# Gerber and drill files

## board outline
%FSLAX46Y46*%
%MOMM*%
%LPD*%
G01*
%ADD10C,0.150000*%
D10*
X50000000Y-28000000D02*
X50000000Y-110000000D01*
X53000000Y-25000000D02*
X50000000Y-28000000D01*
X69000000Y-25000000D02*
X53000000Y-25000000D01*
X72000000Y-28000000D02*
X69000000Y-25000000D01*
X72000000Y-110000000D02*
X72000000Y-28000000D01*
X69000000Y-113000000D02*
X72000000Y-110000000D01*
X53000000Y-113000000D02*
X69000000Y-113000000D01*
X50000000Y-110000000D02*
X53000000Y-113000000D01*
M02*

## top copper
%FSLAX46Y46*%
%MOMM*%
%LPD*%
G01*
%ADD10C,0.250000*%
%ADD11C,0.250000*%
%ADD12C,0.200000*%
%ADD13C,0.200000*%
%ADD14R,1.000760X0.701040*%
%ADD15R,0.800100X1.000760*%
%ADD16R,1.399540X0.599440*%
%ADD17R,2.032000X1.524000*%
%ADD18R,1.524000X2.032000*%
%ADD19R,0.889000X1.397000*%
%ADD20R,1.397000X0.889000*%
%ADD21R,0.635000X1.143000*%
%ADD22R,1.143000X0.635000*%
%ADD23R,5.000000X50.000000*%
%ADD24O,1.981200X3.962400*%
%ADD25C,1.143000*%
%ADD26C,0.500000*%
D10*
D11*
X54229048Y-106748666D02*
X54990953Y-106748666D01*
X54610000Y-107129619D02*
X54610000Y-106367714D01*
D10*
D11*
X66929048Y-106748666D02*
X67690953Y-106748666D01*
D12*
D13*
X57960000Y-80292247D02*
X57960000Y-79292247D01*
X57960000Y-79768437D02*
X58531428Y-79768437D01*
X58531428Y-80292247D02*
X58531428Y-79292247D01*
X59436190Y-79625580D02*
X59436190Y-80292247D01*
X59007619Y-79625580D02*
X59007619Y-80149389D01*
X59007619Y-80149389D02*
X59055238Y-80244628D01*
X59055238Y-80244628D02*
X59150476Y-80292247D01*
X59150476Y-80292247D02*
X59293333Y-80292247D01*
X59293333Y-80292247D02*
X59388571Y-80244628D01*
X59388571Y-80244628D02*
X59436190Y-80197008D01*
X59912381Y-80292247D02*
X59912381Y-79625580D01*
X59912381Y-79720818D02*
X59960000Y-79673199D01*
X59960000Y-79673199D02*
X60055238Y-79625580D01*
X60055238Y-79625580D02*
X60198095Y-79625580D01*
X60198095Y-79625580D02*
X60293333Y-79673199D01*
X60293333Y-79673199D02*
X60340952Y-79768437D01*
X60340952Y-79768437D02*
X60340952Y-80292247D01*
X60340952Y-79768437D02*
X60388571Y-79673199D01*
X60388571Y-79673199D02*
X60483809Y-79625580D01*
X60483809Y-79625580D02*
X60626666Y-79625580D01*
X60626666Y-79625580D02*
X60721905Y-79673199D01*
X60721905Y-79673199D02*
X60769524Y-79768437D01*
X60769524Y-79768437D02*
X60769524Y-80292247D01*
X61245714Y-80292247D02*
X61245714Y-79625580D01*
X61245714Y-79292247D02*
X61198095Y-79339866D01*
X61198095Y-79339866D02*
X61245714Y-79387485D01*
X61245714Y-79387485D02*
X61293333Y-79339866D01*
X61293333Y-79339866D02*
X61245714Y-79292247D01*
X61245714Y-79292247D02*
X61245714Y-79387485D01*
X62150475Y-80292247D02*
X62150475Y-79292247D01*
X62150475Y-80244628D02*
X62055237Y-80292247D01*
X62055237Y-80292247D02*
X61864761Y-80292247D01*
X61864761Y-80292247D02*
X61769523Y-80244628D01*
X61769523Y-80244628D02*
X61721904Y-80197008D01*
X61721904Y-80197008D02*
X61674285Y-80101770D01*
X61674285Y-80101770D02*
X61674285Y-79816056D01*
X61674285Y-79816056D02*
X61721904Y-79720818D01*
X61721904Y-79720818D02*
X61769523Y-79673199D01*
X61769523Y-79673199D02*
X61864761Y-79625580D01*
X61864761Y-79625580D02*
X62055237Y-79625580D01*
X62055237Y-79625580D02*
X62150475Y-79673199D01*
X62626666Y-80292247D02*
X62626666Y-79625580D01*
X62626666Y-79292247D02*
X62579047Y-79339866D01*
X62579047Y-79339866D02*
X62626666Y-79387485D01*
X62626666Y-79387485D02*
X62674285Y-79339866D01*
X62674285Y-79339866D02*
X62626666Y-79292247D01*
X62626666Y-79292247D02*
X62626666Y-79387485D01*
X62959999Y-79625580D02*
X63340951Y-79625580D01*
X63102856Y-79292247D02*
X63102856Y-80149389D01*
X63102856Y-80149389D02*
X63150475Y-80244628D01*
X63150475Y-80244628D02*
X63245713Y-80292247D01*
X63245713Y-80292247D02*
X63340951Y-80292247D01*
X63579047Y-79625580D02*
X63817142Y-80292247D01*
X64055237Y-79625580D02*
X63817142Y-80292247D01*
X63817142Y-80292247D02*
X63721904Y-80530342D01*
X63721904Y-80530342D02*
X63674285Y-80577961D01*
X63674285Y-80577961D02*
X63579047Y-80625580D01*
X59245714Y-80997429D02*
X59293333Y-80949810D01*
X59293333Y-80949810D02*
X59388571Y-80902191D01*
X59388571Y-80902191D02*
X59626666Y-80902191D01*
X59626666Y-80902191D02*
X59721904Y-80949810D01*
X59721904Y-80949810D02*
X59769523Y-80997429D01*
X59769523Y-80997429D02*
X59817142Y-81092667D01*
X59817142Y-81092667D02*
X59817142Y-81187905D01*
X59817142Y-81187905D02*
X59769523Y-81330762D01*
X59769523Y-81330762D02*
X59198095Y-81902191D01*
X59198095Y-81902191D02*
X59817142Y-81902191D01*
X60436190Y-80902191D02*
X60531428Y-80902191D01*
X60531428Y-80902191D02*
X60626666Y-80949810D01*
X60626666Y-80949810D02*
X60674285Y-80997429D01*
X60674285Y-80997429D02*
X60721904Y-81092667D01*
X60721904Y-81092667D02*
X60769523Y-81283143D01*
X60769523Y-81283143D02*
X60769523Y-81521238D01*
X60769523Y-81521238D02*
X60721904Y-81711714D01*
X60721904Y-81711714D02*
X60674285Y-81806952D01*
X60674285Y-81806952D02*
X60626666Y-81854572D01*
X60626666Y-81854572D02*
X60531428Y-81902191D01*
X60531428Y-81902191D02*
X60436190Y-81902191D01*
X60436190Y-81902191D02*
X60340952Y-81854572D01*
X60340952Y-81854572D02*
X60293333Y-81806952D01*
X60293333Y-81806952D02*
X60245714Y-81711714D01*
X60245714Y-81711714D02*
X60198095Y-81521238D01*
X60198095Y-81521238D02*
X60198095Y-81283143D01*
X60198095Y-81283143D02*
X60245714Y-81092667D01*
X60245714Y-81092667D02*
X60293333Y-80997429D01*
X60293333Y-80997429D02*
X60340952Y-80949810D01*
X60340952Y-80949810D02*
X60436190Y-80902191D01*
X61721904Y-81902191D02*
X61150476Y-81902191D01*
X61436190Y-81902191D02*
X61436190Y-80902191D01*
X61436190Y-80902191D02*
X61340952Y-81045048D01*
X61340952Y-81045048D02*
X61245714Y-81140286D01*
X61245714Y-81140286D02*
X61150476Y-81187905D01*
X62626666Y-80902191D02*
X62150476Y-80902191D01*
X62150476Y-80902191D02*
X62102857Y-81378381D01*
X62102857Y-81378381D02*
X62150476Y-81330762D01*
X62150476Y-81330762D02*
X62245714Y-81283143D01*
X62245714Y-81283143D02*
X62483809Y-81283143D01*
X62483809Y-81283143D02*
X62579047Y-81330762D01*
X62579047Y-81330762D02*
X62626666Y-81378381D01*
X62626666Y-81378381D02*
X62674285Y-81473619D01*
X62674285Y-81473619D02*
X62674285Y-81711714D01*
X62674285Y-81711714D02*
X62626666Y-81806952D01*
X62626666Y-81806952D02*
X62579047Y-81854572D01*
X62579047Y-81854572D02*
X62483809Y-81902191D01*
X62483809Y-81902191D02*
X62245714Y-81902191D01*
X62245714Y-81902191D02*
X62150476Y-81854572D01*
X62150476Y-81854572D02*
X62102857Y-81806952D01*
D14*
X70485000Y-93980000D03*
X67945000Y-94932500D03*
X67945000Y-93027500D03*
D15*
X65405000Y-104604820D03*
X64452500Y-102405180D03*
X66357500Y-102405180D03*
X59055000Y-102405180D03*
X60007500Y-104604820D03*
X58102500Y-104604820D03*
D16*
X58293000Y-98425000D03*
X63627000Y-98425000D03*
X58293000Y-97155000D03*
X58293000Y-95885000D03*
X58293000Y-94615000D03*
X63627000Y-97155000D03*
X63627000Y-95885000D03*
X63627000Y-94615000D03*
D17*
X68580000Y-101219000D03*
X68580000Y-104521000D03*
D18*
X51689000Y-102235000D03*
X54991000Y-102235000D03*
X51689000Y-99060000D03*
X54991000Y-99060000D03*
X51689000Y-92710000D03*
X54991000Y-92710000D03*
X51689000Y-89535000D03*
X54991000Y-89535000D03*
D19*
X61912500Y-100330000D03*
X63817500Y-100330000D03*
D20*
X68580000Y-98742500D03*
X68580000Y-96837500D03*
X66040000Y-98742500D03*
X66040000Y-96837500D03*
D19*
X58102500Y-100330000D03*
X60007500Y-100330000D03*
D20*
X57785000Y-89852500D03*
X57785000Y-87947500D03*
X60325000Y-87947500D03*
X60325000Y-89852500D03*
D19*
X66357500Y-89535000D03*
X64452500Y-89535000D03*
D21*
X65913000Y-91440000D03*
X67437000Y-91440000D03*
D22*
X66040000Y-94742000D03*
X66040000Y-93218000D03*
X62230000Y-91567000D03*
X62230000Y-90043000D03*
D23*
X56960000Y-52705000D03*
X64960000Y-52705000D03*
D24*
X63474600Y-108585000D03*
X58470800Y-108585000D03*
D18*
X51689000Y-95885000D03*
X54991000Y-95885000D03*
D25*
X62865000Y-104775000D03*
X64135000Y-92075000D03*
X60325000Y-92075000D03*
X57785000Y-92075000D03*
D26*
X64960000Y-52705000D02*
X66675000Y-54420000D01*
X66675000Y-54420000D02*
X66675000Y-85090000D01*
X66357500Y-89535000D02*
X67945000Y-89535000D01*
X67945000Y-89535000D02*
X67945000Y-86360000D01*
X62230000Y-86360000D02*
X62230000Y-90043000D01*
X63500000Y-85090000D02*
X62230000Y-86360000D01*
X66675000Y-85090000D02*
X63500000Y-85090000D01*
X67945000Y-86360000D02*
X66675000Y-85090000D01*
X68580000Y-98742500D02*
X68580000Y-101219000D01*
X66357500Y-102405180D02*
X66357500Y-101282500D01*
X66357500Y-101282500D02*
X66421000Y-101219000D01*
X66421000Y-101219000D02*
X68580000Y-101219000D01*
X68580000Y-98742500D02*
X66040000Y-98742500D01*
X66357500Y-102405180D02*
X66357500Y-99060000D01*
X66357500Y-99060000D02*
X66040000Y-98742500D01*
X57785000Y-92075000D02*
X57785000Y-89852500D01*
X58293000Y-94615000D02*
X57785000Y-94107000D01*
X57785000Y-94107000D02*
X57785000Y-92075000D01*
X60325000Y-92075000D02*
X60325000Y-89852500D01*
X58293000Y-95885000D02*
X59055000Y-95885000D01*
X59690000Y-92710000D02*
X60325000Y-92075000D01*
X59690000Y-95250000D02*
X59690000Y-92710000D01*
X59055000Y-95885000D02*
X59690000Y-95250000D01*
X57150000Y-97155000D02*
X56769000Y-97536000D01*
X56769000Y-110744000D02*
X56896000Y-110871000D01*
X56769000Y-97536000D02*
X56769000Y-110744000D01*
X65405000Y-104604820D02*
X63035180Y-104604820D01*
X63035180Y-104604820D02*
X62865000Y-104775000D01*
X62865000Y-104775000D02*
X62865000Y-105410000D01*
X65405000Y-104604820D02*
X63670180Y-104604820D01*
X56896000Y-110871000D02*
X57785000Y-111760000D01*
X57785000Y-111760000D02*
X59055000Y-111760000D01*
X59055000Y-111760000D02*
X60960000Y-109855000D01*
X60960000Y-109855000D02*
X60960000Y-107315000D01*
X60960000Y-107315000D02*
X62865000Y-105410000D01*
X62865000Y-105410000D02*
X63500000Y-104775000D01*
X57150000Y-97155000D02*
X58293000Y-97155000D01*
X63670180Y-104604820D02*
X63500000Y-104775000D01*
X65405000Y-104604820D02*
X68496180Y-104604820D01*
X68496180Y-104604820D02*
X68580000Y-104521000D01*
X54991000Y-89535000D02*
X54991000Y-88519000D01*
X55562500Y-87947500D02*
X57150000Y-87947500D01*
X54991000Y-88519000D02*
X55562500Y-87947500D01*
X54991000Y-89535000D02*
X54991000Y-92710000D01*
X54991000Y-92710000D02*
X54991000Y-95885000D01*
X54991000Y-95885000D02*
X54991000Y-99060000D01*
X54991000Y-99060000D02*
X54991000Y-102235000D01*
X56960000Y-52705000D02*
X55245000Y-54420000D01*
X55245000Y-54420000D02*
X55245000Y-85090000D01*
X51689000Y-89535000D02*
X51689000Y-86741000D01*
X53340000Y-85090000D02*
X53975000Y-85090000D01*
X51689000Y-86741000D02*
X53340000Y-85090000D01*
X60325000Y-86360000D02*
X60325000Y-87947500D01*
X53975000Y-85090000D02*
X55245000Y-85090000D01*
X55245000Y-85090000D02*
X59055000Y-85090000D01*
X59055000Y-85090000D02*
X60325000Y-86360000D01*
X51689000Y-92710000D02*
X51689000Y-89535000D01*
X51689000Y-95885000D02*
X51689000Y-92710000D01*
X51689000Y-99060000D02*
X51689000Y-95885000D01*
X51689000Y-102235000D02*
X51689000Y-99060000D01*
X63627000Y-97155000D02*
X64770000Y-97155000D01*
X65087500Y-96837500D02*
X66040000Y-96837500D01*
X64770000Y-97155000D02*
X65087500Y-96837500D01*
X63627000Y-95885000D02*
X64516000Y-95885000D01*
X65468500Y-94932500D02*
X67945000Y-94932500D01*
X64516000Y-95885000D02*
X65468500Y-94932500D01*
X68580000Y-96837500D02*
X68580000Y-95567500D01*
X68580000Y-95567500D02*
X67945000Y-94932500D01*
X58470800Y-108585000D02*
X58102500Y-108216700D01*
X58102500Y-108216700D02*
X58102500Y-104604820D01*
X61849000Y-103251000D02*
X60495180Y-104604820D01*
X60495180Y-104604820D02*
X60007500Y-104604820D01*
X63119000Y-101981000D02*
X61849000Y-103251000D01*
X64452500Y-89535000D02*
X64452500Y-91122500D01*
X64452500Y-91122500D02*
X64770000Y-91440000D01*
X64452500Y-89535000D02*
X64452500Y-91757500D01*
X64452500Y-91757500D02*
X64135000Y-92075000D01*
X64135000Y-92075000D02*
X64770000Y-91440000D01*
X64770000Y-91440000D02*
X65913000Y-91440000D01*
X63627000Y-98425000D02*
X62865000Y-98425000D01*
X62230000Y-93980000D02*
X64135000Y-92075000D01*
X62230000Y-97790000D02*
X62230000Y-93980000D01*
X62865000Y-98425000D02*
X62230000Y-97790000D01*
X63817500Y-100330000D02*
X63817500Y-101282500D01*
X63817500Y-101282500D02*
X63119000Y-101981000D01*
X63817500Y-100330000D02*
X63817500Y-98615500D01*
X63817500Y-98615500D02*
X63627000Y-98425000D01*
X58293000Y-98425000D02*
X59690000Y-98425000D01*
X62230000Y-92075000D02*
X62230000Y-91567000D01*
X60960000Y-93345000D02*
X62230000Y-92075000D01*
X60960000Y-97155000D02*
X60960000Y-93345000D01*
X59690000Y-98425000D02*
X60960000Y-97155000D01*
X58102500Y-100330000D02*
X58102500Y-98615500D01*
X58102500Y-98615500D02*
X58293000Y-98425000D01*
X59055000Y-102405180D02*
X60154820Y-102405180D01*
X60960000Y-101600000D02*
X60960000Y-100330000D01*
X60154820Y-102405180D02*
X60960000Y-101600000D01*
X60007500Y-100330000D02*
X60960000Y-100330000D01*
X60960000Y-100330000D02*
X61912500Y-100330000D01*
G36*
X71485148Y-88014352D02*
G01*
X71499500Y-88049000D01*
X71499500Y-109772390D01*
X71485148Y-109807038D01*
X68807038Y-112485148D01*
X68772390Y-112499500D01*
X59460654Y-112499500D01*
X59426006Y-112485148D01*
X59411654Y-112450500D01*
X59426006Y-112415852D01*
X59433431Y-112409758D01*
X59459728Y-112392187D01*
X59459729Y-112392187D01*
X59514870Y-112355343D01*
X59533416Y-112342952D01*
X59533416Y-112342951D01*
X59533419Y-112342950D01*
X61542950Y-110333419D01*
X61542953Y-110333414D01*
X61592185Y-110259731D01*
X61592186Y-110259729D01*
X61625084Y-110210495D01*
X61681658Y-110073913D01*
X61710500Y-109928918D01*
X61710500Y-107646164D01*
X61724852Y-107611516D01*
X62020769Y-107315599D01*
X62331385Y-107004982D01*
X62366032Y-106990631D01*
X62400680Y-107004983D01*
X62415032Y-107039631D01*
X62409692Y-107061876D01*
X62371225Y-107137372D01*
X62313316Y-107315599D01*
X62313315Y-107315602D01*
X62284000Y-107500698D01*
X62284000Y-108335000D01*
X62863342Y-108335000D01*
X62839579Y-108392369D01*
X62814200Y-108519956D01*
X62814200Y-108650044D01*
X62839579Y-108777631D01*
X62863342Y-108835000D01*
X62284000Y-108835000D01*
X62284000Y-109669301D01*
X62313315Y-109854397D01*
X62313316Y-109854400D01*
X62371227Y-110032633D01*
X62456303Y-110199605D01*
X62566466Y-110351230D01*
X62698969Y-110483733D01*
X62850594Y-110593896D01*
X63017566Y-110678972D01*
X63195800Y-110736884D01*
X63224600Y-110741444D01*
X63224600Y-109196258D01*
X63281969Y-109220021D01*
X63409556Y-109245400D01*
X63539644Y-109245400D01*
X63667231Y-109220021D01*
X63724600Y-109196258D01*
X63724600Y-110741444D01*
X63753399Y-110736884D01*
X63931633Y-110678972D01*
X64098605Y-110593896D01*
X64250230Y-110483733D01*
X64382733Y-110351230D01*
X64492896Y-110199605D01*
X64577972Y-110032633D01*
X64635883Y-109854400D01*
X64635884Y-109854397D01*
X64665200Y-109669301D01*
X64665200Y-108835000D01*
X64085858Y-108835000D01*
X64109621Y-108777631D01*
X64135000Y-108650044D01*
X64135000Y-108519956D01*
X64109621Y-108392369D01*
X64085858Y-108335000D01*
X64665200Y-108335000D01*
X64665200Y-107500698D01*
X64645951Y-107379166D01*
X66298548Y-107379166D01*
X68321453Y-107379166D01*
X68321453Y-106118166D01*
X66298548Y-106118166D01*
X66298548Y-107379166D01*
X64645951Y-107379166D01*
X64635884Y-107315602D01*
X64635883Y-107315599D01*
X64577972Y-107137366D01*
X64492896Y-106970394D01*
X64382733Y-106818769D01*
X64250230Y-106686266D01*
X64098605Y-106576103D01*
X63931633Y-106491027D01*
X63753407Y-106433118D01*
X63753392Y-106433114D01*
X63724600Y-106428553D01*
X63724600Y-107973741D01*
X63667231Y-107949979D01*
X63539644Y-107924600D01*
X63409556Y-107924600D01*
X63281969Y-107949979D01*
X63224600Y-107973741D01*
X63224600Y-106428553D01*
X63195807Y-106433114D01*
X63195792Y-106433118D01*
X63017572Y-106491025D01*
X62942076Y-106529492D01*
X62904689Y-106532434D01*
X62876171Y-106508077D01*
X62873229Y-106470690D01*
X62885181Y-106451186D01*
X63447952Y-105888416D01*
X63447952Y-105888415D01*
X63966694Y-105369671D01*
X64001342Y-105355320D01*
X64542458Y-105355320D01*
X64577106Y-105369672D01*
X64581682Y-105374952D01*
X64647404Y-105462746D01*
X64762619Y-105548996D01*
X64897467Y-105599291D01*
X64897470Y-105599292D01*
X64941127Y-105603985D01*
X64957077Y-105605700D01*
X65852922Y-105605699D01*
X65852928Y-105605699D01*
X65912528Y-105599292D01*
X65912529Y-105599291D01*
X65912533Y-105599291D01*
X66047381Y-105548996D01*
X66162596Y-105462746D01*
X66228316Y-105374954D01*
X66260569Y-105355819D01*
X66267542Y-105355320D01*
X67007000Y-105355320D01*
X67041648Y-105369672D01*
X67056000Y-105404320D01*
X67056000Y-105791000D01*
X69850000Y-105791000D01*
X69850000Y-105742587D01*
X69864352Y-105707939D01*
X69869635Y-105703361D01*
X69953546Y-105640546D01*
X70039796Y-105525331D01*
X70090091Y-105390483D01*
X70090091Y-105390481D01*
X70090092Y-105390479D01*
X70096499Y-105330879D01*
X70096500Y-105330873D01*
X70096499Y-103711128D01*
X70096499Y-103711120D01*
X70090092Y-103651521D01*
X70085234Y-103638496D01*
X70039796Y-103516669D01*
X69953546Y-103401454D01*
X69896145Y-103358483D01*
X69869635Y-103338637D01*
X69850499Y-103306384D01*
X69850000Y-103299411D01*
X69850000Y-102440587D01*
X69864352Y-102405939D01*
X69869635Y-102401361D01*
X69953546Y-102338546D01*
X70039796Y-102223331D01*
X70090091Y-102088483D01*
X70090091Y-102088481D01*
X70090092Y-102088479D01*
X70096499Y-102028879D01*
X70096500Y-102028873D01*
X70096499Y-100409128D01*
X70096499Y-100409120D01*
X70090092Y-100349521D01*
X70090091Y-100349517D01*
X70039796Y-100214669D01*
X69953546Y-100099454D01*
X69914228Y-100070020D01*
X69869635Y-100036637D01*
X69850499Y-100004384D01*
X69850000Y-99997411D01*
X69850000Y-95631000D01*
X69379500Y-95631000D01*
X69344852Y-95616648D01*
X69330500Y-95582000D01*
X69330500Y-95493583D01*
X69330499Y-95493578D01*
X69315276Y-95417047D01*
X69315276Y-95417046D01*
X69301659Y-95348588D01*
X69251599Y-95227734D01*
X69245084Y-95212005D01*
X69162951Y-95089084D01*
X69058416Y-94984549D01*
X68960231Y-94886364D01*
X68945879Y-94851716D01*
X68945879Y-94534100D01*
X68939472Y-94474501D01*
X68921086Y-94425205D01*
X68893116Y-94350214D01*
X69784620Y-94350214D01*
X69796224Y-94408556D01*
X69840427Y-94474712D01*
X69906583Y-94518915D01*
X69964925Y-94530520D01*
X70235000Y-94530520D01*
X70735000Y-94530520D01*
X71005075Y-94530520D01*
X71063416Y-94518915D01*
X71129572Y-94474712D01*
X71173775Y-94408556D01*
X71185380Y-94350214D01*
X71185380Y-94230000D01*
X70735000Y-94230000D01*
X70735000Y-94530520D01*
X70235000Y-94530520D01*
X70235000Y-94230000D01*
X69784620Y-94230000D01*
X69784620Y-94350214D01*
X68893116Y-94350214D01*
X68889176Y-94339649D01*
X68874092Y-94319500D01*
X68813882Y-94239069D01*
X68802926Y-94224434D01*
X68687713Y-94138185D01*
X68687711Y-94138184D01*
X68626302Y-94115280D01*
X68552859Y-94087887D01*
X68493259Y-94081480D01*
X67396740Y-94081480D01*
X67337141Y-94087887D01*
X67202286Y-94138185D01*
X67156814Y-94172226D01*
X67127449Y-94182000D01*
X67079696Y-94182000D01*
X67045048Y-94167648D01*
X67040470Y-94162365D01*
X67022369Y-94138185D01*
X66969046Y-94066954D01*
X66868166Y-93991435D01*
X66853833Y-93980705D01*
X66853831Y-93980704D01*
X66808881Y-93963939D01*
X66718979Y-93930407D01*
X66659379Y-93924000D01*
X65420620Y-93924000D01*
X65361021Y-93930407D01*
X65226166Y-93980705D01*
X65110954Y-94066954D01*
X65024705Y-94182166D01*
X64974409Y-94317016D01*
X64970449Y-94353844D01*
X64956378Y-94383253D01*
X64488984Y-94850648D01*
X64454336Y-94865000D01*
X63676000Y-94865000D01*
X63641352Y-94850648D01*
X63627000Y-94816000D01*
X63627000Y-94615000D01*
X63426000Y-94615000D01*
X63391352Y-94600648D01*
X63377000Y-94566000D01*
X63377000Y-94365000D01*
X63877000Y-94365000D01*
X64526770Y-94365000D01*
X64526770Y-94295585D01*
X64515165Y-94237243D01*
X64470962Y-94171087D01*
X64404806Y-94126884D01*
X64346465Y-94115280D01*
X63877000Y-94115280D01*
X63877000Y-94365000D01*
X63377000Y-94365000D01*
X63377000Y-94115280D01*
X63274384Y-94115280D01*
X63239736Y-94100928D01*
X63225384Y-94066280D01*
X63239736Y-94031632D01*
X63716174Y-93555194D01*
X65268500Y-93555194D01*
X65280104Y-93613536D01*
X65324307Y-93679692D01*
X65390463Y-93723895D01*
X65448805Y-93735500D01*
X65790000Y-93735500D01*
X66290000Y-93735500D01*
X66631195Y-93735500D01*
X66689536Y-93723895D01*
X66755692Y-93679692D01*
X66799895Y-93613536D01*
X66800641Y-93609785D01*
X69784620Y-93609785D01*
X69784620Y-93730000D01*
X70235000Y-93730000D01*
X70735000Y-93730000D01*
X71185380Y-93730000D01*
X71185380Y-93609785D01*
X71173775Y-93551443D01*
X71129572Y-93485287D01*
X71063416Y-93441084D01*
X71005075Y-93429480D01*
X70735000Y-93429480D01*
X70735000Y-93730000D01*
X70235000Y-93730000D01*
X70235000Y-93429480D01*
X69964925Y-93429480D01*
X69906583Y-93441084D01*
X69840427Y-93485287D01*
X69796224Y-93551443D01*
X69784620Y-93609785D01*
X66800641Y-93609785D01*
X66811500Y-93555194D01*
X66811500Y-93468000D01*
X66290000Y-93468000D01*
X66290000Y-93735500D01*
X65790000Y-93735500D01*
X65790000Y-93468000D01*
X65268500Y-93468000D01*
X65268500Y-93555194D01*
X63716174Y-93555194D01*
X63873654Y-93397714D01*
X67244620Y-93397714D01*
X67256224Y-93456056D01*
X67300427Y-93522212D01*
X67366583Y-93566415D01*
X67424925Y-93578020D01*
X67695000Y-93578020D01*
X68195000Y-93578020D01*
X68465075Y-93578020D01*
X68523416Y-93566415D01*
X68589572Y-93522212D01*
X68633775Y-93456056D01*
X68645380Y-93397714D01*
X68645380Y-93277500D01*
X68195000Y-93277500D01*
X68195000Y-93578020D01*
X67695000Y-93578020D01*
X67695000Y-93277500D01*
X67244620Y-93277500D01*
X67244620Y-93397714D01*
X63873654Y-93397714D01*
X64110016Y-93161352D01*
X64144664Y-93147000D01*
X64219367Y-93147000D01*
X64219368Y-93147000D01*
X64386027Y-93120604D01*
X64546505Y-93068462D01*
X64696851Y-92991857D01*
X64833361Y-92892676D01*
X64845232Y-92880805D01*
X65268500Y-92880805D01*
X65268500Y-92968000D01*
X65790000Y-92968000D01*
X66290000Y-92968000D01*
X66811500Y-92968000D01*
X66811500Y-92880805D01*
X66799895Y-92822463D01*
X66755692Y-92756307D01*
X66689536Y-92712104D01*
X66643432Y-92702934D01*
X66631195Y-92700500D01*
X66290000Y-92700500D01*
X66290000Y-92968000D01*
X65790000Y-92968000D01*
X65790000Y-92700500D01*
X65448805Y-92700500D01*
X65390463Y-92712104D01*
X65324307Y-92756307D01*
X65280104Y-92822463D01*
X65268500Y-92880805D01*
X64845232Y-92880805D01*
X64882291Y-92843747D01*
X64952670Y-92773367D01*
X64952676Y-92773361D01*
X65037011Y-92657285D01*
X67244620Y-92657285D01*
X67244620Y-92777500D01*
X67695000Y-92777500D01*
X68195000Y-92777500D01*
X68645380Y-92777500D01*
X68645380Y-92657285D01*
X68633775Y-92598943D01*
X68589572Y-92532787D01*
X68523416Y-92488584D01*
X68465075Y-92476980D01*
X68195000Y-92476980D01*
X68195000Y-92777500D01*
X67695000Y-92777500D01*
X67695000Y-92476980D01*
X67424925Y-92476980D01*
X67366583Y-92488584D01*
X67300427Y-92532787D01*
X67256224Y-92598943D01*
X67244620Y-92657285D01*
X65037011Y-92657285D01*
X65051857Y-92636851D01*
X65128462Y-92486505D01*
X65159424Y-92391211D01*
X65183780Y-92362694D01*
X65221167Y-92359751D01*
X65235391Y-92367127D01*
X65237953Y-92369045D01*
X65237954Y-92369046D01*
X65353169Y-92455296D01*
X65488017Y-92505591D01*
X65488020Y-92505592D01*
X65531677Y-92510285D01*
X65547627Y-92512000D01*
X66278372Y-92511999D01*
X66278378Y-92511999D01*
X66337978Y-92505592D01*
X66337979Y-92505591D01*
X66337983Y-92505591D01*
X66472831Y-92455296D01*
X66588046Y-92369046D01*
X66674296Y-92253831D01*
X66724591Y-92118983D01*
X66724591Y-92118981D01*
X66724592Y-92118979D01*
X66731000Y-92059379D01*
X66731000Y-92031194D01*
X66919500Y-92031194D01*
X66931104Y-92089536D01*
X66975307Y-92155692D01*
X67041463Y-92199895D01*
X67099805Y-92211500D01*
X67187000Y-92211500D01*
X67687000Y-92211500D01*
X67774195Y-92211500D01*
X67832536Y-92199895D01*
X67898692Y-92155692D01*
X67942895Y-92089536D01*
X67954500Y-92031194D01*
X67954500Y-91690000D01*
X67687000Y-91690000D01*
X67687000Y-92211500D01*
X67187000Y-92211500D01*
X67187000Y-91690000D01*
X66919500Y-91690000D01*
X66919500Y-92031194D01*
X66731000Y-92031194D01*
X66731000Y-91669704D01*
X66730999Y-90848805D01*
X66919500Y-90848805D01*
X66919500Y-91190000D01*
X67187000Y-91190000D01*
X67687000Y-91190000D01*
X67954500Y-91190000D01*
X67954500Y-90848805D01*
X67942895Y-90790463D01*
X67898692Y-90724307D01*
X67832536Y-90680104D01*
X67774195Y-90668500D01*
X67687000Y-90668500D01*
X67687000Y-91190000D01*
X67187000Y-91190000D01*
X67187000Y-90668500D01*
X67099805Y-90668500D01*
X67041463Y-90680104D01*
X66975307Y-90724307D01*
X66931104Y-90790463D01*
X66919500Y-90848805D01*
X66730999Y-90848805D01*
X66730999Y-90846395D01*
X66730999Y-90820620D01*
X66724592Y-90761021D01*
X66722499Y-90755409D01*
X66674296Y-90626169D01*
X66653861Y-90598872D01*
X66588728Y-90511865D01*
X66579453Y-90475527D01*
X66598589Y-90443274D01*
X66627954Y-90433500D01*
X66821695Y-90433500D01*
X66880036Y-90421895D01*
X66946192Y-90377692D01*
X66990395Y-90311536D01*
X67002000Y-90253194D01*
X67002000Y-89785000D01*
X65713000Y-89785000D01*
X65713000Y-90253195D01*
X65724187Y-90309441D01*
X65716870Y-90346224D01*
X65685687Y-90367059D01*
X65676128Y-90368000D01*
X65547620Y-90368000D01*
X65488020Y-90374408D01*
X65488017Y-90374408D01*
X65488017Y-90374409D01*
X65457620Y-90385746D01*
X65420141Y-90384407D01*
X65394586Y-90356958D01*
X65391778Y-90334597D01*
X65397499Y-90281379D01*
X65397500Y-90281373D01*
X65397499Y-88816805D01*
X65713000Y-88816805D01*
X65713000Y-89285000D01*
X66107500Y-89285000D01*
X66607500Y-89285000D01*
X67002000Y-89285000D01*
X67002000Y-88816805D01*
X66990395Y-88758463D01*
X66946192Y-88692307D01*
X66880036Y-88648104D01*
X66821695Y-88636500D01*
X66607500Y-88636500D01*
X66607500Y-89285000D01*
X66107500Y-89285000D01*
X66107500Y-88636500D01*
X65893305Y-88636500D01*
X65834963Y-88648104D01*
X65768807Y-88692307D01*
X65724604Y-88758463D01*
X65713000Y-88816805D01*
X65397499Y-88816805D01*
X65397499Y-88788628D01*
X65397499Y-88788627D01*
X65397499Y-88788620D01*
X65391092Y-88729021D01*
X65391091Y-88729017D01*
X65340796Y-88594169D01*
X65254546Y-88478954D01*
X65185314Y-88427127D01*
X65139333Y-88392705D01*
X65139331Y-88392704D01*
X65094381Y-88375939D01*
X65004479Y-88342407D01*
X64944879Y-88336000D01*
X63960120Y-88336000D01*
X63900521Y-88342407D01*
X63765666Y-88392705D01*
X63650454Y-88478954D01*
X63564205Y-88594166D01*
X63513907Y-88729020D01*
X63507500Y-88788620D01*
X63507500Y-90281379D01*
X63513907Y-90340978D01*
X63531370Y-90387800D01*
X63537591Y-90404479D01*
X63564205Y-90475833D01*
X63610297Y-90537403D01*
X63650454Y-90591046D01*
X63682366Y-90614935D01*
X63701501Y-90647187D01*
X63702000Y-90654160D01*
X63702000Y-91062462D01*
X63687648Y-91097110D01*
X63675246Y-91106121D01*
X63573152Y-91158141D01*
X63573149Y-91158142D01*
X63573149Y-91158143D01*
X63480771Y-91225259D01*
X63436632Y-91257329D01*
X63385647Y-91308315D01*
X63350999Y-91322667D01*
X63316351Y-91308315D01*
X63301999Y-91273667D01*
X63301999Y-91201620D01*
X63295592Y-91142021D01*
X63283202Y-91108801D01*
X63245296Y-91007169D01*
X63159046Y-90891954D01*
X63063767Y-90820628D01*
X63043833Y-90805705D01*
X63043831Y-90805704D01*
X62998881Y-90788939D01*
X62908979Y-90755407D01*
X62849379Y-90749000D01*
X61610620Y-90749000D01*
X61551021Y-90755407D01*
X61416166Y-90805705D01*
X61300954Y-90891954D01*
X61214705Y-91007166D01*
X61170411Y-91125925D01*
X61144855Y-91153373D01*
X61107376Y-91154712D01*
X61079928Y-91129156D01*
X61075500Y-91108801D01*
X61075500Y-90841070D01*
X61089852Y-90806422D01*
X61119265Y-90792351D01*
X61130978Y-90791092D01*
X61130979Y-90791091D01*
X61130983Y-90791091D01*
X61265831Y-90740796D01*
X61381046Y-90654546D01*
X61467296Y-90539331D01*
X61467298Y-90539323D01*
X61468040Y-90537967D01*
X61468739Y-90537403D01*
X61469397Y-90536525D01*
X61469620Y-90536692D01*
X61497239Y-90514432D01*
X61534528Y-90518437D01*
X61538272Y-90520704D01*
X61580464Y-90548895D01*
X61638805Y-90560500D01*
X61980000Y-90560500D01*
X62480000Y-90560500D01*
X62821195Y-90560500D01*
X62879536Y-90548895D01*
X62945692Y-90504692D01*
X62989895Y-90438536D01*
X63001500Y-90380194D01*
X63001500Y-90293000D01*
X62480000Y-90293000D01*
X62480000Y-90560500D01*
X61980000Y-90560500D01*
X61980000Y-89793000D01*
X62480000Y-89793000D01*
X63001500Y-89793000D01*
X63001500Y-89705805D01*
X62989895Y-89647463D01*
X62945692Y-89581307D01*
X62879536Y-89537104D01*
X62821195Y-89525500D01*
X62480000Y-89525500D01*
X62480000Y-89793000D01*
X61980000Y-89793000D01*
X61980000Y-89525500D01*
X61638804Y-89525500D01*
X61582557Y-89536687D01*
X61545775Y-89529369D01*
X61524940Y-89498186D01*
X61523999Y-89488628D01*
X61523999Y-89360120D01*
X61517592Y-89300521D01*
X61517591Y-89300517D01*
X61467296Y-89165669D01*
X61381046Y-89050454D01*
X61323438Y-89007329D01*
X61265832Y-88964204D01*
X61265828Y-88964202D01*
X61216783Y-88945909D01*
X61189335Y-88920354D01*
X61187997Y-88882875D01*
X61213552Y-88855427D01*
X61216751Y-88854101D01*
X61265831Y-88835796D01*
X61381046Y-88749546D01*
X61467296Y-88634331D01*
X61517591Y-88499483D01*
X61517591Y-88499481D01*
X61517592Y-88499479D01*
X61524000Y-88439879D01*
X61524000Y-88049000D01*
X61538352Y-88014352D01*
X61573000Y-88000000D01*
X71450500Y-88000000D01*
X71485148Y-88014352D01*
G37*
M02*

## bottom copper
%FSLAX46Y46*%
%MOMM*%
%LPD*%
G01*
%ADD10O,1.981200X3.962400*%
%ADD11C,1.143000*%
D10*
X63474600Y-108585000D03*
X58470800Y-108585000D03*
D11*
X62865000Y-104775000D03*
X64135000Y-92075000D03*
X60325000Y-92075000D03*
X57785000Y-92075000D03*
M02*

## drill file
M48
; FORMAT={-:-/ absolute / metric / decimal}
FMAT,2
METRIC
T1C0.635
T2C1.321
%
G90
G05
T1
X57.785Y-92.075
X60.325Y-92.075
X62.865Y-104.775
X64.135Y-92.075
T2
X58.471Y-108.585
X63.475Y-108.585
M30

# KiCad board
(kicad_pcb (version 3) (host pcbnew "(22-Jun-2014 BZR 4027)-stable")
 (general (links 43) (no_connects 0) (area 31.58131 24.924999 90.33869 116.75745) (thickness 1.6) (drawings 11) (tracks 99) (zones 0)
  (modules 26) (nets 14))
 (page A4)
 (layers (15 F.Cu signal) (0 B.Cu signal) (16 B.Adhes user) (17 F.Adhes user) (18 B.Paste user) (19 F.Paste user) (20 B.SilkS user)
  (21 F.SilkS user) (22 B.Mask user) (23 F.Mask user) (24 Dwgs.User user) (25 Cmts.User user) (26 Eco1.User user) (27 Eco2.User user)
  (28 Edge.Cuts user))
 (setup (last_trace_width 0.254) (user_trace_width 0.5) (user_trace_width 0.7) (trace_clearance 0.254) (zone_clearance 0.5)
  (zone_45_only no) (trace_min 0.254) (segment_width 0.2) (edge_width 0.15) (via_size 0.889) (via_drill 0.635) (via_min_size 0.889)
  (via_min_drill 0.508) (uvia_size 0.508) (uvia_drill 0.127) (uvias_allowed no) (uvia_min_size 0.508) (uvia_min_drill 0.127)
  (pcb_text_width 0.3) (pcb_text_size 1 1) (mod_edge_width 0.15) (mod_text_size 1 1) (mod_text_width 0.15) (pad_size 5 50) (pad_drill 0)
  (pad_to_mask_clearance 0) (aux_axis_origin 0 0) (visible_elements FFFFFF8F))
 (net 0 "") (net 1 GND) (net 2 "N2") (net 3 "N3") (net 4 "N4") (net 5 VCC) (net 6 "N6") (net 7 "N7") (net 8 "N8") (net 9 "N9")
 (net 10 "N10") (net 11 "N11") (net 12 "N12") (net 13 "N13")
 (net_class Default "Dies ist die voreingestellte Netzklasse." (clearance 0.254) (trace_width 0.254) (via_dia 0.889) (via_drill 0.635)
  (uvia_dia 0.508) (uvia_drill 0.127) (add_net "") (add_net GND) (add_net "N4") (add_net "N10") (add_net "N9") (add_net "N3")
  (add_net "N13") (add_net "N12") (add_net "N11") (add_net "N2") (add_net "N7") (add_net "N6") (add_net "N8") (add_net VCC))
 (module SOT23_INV (layer F.Cu) (at 69.215 93.98 270)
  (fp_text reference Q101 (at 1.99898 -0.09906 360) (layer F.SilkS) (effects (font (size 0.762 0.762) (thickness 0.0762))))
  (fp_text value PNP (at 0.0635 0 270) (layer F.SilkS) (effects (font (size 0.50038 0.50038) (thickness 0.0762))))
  (pad 3 smd rect (at 0 -1.27 270) (size 0.70104 1.00076) (layers F.Cu F.Paste F.Mask) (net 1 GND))
  (pad 1 smd rect (at 0.9525 1.27 270) (size 0.70104 1.00076) (layers F.Cu F.Paste F.Mask) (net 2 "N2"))
  (pad 2 smd rect (at -0.9525 1.27 270) (size 0.70104 1.00076) (layers F.Cu F.Paste F.Mask) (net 1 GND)))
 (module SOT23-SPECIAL (layer F.Cu) (at 65.405 103.505 180)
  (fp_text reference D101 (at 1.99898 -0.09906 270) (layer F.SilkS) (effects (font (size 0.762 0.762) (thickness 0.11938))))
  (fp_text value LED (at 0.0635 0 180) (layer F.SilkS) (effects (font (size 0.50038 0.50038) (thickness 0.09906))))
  (pad 2 smd rect (at 0 -1.09982 180) (size 0.8001 1.00076) (layers F.Cu F.Paste F.Mask) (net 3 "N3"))
  (pad 3 smd rect (at 0.9525 1.09982 180) (size 0.8001 1.00076) (layers F.Cu F.Paste F.Mask))
  (pad 1 smd rect (at -0.9525 1.09982 180) (size 0.8001 1.00076) (layers F.Cu F.Paste F.Mask) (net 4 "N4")))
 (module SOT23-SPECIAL (layer F.Cu) (at 59.055 103.505)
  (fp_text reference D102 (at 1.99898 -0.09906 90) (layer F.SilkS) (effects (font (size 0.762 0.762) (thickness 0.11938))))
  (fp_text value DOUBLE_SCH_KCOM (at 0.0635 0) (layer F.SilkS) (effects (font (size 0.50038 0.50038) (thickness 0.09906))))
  (pad 2 smd rect (at 0 -1.09982) (size 0.8001 1.00076) (layers F.Cu F.Paste F.Mask) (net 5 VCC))
  (pad 3 smd rect (at 0.9525 1.09982) (size 0.8001 1.00076) (layers F.Cu F.Paste F.Mask) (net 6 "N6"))
  (pad 1 smd rect (at -0.9525 1.09982) (size 0.8001 1.00076) (layers F.Cu F.Paste F.Mask) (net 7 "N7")))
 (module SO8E (layer F.Cu) (at 60.96 96.52 90)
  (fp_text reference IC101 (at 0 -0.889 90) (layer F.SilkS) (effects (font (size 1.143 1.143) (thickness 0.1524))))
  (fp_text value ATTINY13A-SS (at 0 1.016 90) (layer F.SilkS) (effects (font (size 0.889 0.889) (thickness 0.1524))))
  (pad 8 smd rect (at -1.905 -2.667 90) (size 0.59944 1.39954) (layers F.Cu F.Paste F.Mask) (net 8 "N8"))
  (pad 1 smd rect (at -1.905 2.667 90) (size 0.59944 1.39954) (layers F.Cu F.Paste F.Mask) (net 6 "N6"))
  (pad 7 smd rect (at -0.635 -2.667 90) (size 0.59944 1.39954) (layers F.Cu F.Paste F.Mask) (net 3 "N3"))
  (pad 6 smd rect (at 0.635 -2.667 90) (size 0.59944 1.39954) (layers F.Cu F.Paste F.Mask) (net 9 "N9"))
  (pad 5 smd rect (at 1.905 -2.667 90) (size 0.59944 1.39954) (layers F.Cu F.Paste F.Mask) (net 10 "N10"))
  (pad 2 smd rect (at -0.635 2.667 90) (size 0.59944 1.39954) (layers F.Cu F.Paste F.Mask) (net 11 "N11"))
  (pad 3 smd rect (at 0.635 2.667 90) (size 0.59944 1.39954) (layers F.Cu F.Paste F.Mask) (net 2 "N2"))
  (pad 4 smd rect (at 1.905 2.667 90) (size 0.59944 1.39954) (layers F.Cu F.Paste F.Mask) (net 1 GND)))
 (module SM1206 (layer F.Cu) (at 68.58 102.87 270)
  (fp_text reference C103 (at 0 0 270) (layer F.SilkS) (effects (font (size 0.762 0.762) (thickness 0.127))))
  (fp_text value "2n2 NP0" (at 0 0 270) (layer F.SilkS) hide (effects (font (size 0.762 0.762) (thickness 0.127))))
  (pad 1 smd rect (at -1.651 0 270) (size 1.524 2.032) (layers F.Cu F.Paste F.Mask) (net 4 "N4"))
  (pad 2 smd rect (at 1.651 0 270) (size 1.524 2.032) (layers F.Cu F.Paste F.Mask) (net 3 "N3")))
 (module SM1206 (layer F.Cu) (at 53.34 102.235)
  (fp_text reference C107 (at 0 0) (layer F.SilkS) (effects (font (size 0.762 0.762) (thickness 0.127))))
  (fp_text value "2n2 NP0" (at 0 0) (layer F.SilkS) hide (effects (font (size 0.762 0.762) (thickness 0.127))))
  (pad 1 smd rect (at -1.651 0) (size 1.524 2.032) (layers F.Cu F.Paste F.Mask) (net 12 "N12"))
  (pad 2 smd rect (at 1.651 0) (size 1.524 2.032) (layers F.Cu F.Paste F.Mask) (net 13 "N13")))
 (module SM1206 (layer F.Cu) (at 53.34 99.06)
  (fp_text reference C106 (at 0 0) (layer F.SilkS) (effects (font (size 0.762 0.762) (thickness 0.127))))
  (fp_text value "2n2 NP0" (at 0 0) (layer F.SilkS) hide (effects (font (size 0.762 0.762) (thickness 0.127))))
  (pad 1 smd rect (at -1.651 0) (size 1.524 2.032) (layers F.Cu F.Paste F.Mask) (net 12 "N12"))
  (pad 2 smd rect (at 1.651 0) (size 1.524 2.032) (layers F.Cu F.Paste F.Mask) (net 13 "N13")))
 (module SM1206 (layer F.Cu) (at 53.34 92.71)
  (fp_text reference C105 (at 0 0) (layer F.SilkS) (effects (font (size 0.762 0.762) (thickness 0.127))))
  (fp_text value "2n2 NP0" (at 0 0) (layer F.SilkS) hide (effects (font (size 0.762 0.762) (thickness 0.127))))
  (pad 1 smd rect (at -1.651 0) (size 1.524 2.032) (layers F.Cu F.Paste F.Mask) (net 12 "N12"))
  (pad 2 smd rect (at 1.651 0) (size 1.524 2.032) (layers F.Cu F.Paste F.Mask) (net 13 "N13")))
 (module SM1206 (layer F.Cu) (at 53.34 89.535)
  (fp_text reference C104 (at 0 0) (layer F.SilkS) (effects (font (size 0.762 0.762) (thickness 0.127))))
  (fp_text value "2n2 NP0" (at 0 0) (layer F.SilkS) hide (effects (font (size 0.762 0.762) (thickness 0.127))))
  (pad 1 smd rect (at -1.651 0) (size 1.524 2.032) (layers F.Cu F.Paste F.Mask) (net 12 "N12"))
  (pad 2 smd rect (at 1.651 0) (size 1.524 2.032) (layers F.Cu F.Paste F.Mask) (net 13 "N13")))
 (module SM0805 (layer F.Cu) (at 62.865 100.33)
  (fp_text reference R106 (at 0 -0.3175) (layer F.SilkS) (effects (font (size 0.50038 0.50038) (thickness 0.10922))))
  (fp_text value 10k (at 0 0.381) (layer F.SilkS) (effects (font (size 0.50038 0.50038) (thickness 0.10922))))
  (pad 1 smd rect (at -0.9525 0) (size 0.889 1.397) (layers F.Cu F.Paste F.Mask) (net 5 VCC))
  (pad 2 smd rect (at 0.9525 0) (size 0.889 1.397) (layers F.Cu F.Paste F.Mask) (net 6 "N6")))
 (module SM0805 (layer F.Cu) (at 68.58 97.79 90)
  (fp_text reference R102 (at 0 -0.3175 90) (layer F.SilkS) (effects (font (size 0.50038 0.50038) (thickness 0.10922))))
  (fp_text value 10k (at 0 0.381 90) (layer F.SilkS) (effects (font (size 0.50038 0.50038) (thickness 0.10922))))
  (pad 1 smd rect (at -0.9525 0 90) (size 0.889 1.397) (layers F.Cu F.Paste F.Mask) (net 4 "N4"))
  (pad 2 smd rect (at 0.9525 0 90) (size 0.889 1.397) (layers F.Cu F.Paste F.Mask) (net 2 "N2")))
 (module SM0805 (layer F.Cu) (at 66.04 97.79 90)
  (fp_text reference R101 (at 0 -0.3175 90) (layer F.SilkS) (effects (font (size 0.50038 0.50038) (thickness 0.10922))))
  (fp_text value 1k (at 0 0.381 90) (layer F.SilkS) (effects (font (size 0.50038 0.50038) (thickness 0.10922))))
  (pad 1 smd rect (at -0.9525 0 90) (size 0.889 1.397) (layers F.Cu F.Paste F.Mask) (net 4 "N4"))
  (pad 2 smd rect (at 0.9525 0 90) (size 0.889 1.397) (layers F.Cu F.Paste F.Mask) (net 11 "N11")))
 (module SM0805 (layer F.Cu) (at 59.055 100.33)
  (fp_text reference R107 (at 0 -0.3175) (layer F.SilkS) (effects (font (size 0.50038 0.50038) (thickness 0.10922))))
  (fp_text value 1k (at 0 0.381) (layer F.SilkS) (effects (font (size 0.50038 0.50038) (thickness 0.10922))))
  (pad 1 smd rect (at -0.9525 0) (size 0.889 1.397) (layers F.Cu F.Paste F.Mask) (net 8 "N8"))
  (pad 2 smd rect (at 0.9525 0) (size 0.889 1.397) (layers F.Cu F.Paste F.Mask) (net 5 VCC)))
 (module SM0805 (layer F.Cu) (at 57.785 88.9 90)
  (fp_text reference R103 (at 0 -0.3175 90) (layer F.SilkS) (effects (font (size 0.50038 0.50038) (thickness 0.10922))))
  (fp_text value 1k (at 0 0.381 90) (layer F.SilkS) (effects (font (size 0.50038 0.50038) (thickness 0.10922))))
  (pad 1 smd rect (at -0.9525 0 90) (size 0.889 1.397) (layers F.Cu F.Paste F.Mask) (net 10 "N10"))
  (pad 2 smd rect (at 0.9525 0 90) (size 0.889 1.397) (layers F.Cu F.Paste F.Mask) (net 13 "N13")))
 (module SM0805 (layer F.Cu) (at 60.325 88.9 270)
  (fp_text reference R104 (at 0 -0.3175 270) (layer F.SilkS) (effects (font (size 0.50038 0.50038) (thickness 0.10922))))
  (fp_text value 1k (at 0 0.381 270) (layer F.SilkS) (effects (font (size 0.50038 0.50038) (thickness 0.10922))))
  (pad 1 smd rect (at -0.9525 0 270) (size 0.889 1.397) (layers F.Cu F.Paste F.Mask) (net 12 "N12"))
  (pad 2 smd rect (at 0.9525 0 270) (size 0.889 1.397) (layers F.Cu F.Paste F.Mask) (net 9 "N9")))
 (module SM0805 (layer F.Cu) (at 65.405 89.535 180)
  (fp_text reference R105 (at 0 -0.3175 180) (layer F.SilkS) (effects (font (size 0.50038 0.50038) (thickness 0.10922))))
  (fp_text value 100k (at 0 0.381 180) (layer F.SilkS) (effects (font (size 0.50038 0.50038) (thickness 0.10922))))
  (pad 1 smd rect (at -0.9525 0 180) (size 0.889 1.397) (layers F.Cu F.Paste F.Mask) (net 1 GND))
  (pad 2 smd rect (at 0.9525 0 180) (size 0.889 1.397) (layers F.Cu F.Paste F.Mask) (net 6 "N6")))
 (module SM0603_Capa (layer F.Cu) (at 66.675 91.44)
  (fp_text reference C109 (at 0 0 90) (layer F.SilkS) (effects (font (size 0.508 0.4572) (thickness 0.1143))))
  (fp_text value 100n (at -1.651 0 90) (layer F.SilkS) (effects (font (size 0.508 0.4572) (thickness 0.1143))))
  (pad 1 smd rect (at -0.762 0) (size 0.635 1.143) (layers F.Cu F.Paste F.Mask) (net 6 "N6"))
  (pad 2 smd rect (at 0.762 0) (size 0.635 1.143) (layers F.Cu F.Paste F.Mask) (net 1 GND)))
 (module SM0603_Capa (layer F.Cu) (at 66.04 93.98 90)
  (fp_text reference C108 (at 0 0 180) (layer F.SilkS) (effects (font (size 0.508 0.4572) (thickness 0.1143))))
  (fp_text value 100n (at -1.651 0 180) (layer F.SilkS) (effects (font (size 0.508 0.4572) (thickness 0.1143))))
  (pad 1 smd rect (at -0.762 0 90) (size 0.635 1.143) (layers F.Cu F.Paste F.Mask) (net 2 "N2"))
  (pad 2 smd rect (at 0.762 0 90) (size 0.635 1.143) (layers F.Cu F.Paste F.Mask) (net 1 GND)))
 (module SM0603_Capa (layer F.Cu) (at 62.23 90.805 90)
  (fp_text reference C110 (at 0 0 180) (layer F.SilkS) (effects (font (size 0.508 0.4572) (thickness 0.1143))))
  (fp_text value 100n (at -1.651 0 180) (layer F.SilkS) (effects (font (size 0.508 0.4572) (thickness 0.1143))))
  (pad 1 smd rect (at -0.762 0 90) (size 0.635 1.143) (layers F.Cu F.Paste F.Mask) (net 8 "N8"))
  (pad 2 smd rect (at 0.762 0 90) (size 0.635 1.143) (layers F.Cu F.Paste F.Mask) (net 1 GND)))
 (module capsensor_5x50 (layer F.Cu) (at 60.96 52.705)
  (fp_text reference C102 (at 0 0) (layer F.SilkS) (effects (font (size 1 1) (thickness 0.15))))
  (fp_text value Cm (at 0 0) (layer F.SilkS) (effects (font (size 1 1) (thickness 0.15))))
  (pad 1 smd rect (at -4 0) (size 5 50) (layers F.Cu F.Paste F.Mask) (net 12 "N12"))
  (pad 2 smd rect (at 4 0) (size 5 50) (layers F.Cu F.Paste F.Mask) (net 1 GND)))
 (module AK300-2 (layer F.Cu) (at 60.96 108.585 180)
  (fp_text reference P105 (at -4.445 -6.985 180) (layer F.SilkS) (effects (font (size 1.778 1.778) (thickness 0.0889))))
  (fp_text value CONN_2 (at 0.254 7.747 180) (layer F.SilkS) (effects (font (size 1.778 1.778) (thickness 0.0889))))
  (pad 1 thru_hole oval (at -2.5146 0 180) (size 1.9812 3.9624) (drill 1.3208) (layers *.Cu F.Paste F.SilkS F.Mask) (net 1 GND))
  (pad 2 thru_hole oval (at 2.4892 0 180) (size 1.9812 3.9624) (drill 1.3208) (layers *.Cu F.Paste F.SilkS F.Mask) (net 7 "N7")))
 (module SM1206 (layer F.Cu) (at 53.34 95.885)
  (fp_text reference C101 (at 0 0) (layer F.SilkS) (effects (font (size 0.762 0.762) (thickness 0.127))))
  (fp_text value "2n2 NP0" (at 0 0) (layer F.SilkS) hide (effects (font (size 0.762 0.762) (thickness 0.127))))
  (pad 1 smd rect (at -1.651 0) (size 1.524 2.032) (layers F.Cu F.Paste F.Mask) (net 12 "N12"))
  (pad 2 smd rect (at 1.651 0) (size 1.524 2.032) (layers F.Cu F.Paste F.Mask) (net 13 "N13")))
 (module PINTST (layer F.Cu) (at 62.865 104.775)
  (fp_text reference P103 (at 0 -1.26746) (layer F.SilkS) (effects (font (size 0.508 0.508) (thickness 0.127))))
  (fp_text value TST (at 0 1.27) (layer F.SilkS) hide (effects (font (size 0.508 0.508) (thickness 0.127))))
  (pad 1 thru_hole circle (at 0 0) (size 1.143 1.143) (drill 0.635) (layers *.Cu *.Mask F.SilkS) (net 3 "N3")))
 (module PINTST (layer F.Cu) (at 64.135 92.075)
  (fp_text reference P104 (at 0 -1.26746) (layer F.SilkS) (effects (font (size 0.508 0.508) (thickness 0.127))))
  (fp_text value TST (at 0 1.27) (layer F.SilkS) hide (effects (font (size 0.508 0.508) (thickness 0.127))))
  (pad 1 thru_hole circle (at 0 0) (size 1.143 1.143) (drill 0.635) (layers *.Cu *.Mask F.SilkS) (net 6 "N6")))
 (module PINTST (layer F.Cu) (at 60.325 92.075)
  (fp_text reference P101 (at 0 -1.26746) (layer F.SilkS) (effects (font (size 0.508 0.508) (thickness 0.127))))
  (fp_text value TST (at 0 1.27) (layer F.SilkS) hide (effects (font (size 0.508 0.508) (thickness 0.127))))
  (pad 1 thru_hole circle (at 0 0) (size 1.143 1.143) (drill 0.635) (layers *.Cu *.Mask F.SilkS) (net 9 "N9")))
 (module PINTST (layer F.Cu) (at 57.785 92.075)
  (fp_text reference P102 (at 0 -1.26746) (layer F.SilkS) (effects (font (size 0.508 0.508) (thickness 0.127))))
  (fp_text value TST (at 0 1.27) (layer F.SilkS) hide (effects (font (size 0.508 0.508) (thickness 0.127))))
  (pad 1 thru_hole circle (at 0 0) (size 1.143 1.143) (drill 0.635) (layers *.Cu *.Mask F.SilkS) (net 10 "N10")))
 (gr_line (start 50 28) (end 50 110) (angle 90) (layer Edge.Cuts) (width 0.15))
 (gr_line (start 53 25) (end 50 28) (angle 90) (layer Edge.Cuts) (width 0.15))
 (gr_line (start 69 25) (end 53 25) (angle 90) (layer Edge.Cuts) (width 0.15))
 (gr_line (start 72 28) (end 69 25) (angle 90) (layer Edge.Cuts) (width 0.15))
 (gr_line (start 72 110) (end 72 28) (angle 90) (layer Edge.Cuts) (width 0.15))
 (gr_line (start 69 113) (end 72 110) (angle 90) (layer Edge.Cuts) (width 0.15))
 (gr_line (start 53 113) (end 69 113) (angle 90) (layer Edge.Cuts) (width 0.15))
 (gr_line (start 50 110) (end 53 113) (angle 90) (layer Edge.Cuts) (width 0.15))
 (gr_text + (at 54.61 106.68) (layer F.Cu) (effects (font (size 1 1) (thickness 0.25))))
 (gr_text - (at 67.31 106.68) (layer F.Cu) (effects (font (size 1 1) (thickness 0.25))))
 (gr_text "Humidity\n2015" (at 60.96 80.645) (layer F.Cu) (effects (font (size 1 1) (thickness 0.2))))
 (segment (start 64.96 52.705) (end 66.675 54.42) (width 0.5) (layer F.Cu) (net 1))
 (segment (start 66.675 54.42) (end 66.675 85.09) (width 0.5) (layer F.Cu) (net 1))
 (segment (start 66.3575 89.535) (end 67.945 89.535) (width 0.5) (layer F.Cu) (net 1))
 (segment (start 67.945 89.535) (end 67.945 86.36) (width 0.5) (layer F.Cu) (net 1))
 (segment (start 62.23 86.36) (end 62.23 90.043) (width 0.5) (layer F.Cu) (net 1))
 (segment (start 63.5 85.09) (end 62.23 86.36) (width 0.5) (layer F.Cu) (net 1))
 (segment (start 66.675 85.09) (end 63.5 85.09) (width 0.5) (layer F.Cu) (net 1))
 (segment (start 67.945 86.36) (end 66.675 85.09) (width 0.5) (layer F.Cu) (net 1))
 (segment (start 68.58 98.7425) (end 68.58 101.219) (width 0.5) (layer F.Cu) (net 4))
 (segment (start 66.3575 102.40518) (end 66.3575 101.2825) (width 0.5) (layer F.Cu) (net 4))
 (segment (start 66.3575 101.2825) (end 66.421 101.219) (width 0.5) (layer F.Cu) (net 4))
 (segment (start 66.421 101.219) (end 68.58 101.219) (width 0.5) (layer F.Cu) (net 4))
 (segment (start 68.58 98.7425) (end 66.04 98.7425) (width 0.5) (layer F.Cu) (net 4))
 (segment (start 66.3575 102.40518) (end 66.3575 99.06) (width 0.5) (layer F.Cu) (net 4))
 (segment (start 66.3575 99.06) (end 66.04 98.7425) (width 0.5) (layer F.Cu) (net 4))
 (segment (start 57.785 92.075) (end 57.785 89.8525) (width 0.5) (layer F.Cu) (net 10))
 (segment (start 58.293 94.615) (end 57.785 94.107) (width 0.5) (layer F.Cu) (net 10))
 (segment (start 57.785 94.107) (end 57.785 92.075) (width 0.5) (layer F.Cu) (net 10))
 (segment (start 60.325 92.075) (end 60.325 89.8525) (width 0.5) (layer F.Cu) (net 9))
 (segment (start 58.293 95.885) (end 59.055 95.885) (width 0.5) (layer F.Cu) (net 9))
 (segment (start 59.69 92.71) (end 60.325 92.075) (width 0.5) (layer F.Cu) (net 9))
 (segment (start 59.69 95.25) (end 59.69 92.71) (width 0.5) (layer F.Cu) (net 9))
 (segment (start 59.055 95.885) (end 59.69 95.25) (width 0.5) (layer F.Cu) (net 9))
 (segment (start 57.15 97.155) (end 56.769 97.536) (width 0.5) (layer F.Cu) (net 3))
 (segment (start 56.769 110.744) (end 56.896 110.871) (width 0.5) (layer F.Cu) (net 3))
 (segment (start 56.769 97.536) (end 56.769 110.744) (width 0.5) (layer F.Cu) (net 3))
 (segment (start 65.405 104.60482) (end 63.03518 104.60482) (width 0.5) (layer F.Cu) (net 3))
 (segment (start 63.03518 104.60482) (end 62.865 104.775) (width 0.5) (layer F.Cu) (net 3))
 (segment (start 62.865 104.775) (end 62.865 105.41) (width 0.5) (layer F.Cu) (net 3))
 (segment (start 65.405 104.60482) (end 63.67018 104.60482) (width 0.5) (layer F.Cu) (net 3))
 (segment (start 56.896 110.871) (end 57.785 111.76) (width 0.5) (layer F.Cu) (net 3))
 (segment (start 57.785 111.76) (end 59.055 111.76) (width 0.5) (layer F.Cu) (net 3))
 (segment (start 59.055 111.76) (end 60.96 109.855) (width 0.5) (layer F.Cu) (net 3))
 (segment (start 60.96 109.855) (end 60.96 107.315) (width 0.5) (layer F.Cu) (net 3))
 (segment (start 60.96 107.315) (end 62.865 105.41) (width 0.5) (layer F.Cu) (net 3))
 (segment (start 62.865 105.41) (end 63.5 104.775) (width 0.5) (layer F.Cu) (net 3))
 (segment (start 57.15 97.155) (end 58.293 97.155) (width 0.5) (layer F.Cu) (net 3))
 (segment (start 63.67018 104.60482) (end 63.5 104.775) (width 0.5) (layer F.Cu) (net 3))
 (segment (start 65.405 104.60482) (end 68.49618 104.60482) (width 0.5) (layer F.Cu) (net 3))
 (segment (start 68.49618 104.60482) (end 68.58 104.521) (width 0.5) (layer F.Cu) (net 3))
 (segment (start 54.991 89.535) (end 54.991 88.519) (width 0.5) (layer F.Cu) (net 13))
 (segment (start 55.5625 87.9475) (end 57.15 87.9475) (width 0.5) (layer F.Cu) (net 13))
 (segment (start 54.991 88.519) (end 55.5625 87.9475) (width 0.5) (layer F.Cu) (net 13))
 (segment (start 54.991 89.535) (end 54.991 92.71) (width 0.5) (layer F.Cu) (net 13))
 (segment (start 54.991 92.71) (end 54.991 95.885) (width 0.5) (layer F.Cu) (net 13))
 (segment (start 54.991 95.885) (end 54.991 99.06) (width 0.5) (layer F.Cu) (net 13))
 (segment (start 54.991 99.06) (end 54.991 102.235) (width 0.5) (layer F.Cu) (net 13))
 (segment (start 56.96 52.705) (end 55.245 54.42) (width 0.5) (layer F.Cu) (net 12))
 (segment (start 55.245 54.42) (end 55.245 85.09) (width 0.5) (layer F.Cu) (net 12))
 (segment (start 51.689 89.535) (end 51.689 86.741) (width 0.5) (layer F.Cu) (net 12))
 (segment (start 53.34 85.09) (end 53.975 85.09) (width 0.5) (layer F.Cu) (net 12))
 (segment (start 51.689 86.741) (end 53.34 85.09) (width 0.5) (layer F.Cu) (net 12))
 (segment (start 60.325 86.36) (end 60.325 87.9475) (width 0.5) (layer F.Cu) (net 12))
 (segment (start 53.975 85.09) (end 55.245 85.09) (width 0.5) (layer F.Cu) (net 12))
 (segment (start 55.245 85.09) (end 59.055 85.09) (width 0.5) (layer F.Cu) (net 12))
 (segment (start 59.055 85.09) (end 60.325 86.36) (width 0.5) (layer F.Cu) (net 12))
 (segment (start 51.689 92.71) (end 51.689 89.535) (width 0.5) (layer F.Cu) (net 12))
 (segment (start 51.689 95.885) (end 51.689 92.71) (width 0.5) (layer F.Cu) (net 12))
 (segment (start 51.689 99.06) (end 51.689 95.885) (width 0.5) (layer F.Cu) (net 12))
 (segment (start 51.689 102.235) (end 51.689 99.06) (width 0.5) (layer F.Cu) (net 12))
 (segment (start 63.627 97.155) (end 64.77 97.155) (width 0.5) (layer F.Cu) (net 11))
 (segment (start 65.0875 96.8375) (end 66.04 96.8375) (width 0.5) (layer F.Cu) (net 11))
 (segment (start 64.77 97.155) (end 65.0875 96.8375) (width 0.5) (layer F.Cu) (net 11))
 (segment (start 63.627 95.885) (end 64.516 95.885) (width 0.5) (layer F.Cu) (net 2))
 (segment (start 65.4685 94.9325) (end 67.945 94.9325) (width 0.5) (layer F.Cu) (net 2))
 (segment (start 64.516 95.885) (end 65.4685 94.9325) (width 0.5) (layer F.Cu) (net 2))
 (segment (start 68.58 96.8375) (end 68.58 95.5675) (width 0.5) (layer F.Cu) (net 2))
 (segment (start 68.58 95.5675) (end 67.945 94.9325) (width 0.5) (layer F.Cu) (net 2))
 (segment (start 58.4708 108.585) (end 58.1025 108.2167) (width 0.5) (layer F.Cu) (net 7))
 (segment (start 58.1025 108.2167) (end 58.1025 104.60482) (width 0.5) (layer F.Cu) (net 7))
 (segment (start 61.849 103.251) (end 60.49518 104.60482) (width 0.5) (layer F.Cu) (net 6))
 (segment (start 60.49518 104.60482) (end 60.0075 104.60482) (width 0.5) (layer F.Cu) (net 6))
 (segment (start 63.119 101.981) (end 61.849 103.251) (width 0.5) (layer F.Cu) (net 6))
 (segment (start 64.4525 89.535) (end 64.4525 91.1225) (width 0.5) (layer F.Cu) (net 6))
 (segment (start 64.4525 91.1225) (end 64.77 91.44) (width 0.5) (layer F.Cu) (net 6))
 (segment (start 64.4525 89.535) (end 64.4525 91.7575) (width 0.5) (layer F.Cu) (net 6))
 (segment (start 64.4525 91.7575) (end 64.135 92.075) (width 0.5) (layer F.Cu) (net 6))
 (segment (start 64.135 92.075) (end 64.77 91.44) (width 0.5) (layer F.Cu) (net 6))
 (segment (start 64.77 91.44) (end 65.913 91.44) (width 0.5) (layer F.Cu) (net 6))
 (segment (start 63.627 98.425) (end 62.865 98.425) (width 0.5) (layer F.Cu) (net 6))
 (segment (start 62.23 93.98) (end 64.135 92.075) (width 0.5) (layer F.Cu) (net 6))
 (segment (start 62.23 97.79) (end 62.23 93.98) (width 0.5) (layer F.Cu) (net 6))
 (segment (start 62.865 98.425) (end 62.23 97.79) (width 0.5) (layer F.Cu) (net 6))
 (segment (start 63.8175 100.33) (end 63.8175 101.2825) (width 0.5) (layer F.Cu) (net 6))
 (segment (start 63.8175 101.2825) (end 63.119 101.981) (width 0.5) (layer F.Cu) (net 6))
 (segment (start 63.8175 100.33) (end 63.8175 98.6155) (width 0.5) (layer F.Cu) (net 6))
 (segment (start 63.8175 98.6155) (end 63.627 98.425) (width 0.5) (layer F.Cu) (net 6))
 (segment (start 58.293 98.425) (end 59.69 98.425) (width 0.5) (layer F.Cu) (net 8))
 (segment (start 62.23 92.075) (end 62.23 91.567) (width 0.5) (layer F.Cu) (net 8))
 (segment (start 60.96 93.345) (end 62.23 92.075) (width 0.5) (layer F.Cu) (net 8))
 (segment (start 60.96 97.155) (end 60.96 93.345) (width 0.5) (layer F.Cu) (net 8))
 (segment (start 59.69 98.425) (end 60.96 97.155) (width 0.5) (layer F.Cu) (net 8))
 (segment (start 58.1025 100.33) (end 58.1025 98.6155) (width 0.5) (layer F.Cu) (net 8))
 (segment (start 58.1025 98.6155) (end 58.293 98.425) (width 0.5) (layer F.Cu) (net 8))
 (segment (start 59.055 102.40518) (end 60.15482 102.40518) (width 0.5) (layer F.Cu) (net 5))
 (segment (start 60.96 101.6) (end 60.96 100.33) (width 0.5) (layer F.Cu) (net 5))
 (segment (start 60.15482 102.40518) (end 60.96 101.6) (width 0.5) (layer F.Cu) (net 5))
 (segment (start 60.0075 100.33) (end 60.96 100.33) (width 0.5) (layer F.Cu) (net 5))
 (segment (start 60.96 100.33) (end 61.9125 100.33) (width 0.5) (layer F.Cu) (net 5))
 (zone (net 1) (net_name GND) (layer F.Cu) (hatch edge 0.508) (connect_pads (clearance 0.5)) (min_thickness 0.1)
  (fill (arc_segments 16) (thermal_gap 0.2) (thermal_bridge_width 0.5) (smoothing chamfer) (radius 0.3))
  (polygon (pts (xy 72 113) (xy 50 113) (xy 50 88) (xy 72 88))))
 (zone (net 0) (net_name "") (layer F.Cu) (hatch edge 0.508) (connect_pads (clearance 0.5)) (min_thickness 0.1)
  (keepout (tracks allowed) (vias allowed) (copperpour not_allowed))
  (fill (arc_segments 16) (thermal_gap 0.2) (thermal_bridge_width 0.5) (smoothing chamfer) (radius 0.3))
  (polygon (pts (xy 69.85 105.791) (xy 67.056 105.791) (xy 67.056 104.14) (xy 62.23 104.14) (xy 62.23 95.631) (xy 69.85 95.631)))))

